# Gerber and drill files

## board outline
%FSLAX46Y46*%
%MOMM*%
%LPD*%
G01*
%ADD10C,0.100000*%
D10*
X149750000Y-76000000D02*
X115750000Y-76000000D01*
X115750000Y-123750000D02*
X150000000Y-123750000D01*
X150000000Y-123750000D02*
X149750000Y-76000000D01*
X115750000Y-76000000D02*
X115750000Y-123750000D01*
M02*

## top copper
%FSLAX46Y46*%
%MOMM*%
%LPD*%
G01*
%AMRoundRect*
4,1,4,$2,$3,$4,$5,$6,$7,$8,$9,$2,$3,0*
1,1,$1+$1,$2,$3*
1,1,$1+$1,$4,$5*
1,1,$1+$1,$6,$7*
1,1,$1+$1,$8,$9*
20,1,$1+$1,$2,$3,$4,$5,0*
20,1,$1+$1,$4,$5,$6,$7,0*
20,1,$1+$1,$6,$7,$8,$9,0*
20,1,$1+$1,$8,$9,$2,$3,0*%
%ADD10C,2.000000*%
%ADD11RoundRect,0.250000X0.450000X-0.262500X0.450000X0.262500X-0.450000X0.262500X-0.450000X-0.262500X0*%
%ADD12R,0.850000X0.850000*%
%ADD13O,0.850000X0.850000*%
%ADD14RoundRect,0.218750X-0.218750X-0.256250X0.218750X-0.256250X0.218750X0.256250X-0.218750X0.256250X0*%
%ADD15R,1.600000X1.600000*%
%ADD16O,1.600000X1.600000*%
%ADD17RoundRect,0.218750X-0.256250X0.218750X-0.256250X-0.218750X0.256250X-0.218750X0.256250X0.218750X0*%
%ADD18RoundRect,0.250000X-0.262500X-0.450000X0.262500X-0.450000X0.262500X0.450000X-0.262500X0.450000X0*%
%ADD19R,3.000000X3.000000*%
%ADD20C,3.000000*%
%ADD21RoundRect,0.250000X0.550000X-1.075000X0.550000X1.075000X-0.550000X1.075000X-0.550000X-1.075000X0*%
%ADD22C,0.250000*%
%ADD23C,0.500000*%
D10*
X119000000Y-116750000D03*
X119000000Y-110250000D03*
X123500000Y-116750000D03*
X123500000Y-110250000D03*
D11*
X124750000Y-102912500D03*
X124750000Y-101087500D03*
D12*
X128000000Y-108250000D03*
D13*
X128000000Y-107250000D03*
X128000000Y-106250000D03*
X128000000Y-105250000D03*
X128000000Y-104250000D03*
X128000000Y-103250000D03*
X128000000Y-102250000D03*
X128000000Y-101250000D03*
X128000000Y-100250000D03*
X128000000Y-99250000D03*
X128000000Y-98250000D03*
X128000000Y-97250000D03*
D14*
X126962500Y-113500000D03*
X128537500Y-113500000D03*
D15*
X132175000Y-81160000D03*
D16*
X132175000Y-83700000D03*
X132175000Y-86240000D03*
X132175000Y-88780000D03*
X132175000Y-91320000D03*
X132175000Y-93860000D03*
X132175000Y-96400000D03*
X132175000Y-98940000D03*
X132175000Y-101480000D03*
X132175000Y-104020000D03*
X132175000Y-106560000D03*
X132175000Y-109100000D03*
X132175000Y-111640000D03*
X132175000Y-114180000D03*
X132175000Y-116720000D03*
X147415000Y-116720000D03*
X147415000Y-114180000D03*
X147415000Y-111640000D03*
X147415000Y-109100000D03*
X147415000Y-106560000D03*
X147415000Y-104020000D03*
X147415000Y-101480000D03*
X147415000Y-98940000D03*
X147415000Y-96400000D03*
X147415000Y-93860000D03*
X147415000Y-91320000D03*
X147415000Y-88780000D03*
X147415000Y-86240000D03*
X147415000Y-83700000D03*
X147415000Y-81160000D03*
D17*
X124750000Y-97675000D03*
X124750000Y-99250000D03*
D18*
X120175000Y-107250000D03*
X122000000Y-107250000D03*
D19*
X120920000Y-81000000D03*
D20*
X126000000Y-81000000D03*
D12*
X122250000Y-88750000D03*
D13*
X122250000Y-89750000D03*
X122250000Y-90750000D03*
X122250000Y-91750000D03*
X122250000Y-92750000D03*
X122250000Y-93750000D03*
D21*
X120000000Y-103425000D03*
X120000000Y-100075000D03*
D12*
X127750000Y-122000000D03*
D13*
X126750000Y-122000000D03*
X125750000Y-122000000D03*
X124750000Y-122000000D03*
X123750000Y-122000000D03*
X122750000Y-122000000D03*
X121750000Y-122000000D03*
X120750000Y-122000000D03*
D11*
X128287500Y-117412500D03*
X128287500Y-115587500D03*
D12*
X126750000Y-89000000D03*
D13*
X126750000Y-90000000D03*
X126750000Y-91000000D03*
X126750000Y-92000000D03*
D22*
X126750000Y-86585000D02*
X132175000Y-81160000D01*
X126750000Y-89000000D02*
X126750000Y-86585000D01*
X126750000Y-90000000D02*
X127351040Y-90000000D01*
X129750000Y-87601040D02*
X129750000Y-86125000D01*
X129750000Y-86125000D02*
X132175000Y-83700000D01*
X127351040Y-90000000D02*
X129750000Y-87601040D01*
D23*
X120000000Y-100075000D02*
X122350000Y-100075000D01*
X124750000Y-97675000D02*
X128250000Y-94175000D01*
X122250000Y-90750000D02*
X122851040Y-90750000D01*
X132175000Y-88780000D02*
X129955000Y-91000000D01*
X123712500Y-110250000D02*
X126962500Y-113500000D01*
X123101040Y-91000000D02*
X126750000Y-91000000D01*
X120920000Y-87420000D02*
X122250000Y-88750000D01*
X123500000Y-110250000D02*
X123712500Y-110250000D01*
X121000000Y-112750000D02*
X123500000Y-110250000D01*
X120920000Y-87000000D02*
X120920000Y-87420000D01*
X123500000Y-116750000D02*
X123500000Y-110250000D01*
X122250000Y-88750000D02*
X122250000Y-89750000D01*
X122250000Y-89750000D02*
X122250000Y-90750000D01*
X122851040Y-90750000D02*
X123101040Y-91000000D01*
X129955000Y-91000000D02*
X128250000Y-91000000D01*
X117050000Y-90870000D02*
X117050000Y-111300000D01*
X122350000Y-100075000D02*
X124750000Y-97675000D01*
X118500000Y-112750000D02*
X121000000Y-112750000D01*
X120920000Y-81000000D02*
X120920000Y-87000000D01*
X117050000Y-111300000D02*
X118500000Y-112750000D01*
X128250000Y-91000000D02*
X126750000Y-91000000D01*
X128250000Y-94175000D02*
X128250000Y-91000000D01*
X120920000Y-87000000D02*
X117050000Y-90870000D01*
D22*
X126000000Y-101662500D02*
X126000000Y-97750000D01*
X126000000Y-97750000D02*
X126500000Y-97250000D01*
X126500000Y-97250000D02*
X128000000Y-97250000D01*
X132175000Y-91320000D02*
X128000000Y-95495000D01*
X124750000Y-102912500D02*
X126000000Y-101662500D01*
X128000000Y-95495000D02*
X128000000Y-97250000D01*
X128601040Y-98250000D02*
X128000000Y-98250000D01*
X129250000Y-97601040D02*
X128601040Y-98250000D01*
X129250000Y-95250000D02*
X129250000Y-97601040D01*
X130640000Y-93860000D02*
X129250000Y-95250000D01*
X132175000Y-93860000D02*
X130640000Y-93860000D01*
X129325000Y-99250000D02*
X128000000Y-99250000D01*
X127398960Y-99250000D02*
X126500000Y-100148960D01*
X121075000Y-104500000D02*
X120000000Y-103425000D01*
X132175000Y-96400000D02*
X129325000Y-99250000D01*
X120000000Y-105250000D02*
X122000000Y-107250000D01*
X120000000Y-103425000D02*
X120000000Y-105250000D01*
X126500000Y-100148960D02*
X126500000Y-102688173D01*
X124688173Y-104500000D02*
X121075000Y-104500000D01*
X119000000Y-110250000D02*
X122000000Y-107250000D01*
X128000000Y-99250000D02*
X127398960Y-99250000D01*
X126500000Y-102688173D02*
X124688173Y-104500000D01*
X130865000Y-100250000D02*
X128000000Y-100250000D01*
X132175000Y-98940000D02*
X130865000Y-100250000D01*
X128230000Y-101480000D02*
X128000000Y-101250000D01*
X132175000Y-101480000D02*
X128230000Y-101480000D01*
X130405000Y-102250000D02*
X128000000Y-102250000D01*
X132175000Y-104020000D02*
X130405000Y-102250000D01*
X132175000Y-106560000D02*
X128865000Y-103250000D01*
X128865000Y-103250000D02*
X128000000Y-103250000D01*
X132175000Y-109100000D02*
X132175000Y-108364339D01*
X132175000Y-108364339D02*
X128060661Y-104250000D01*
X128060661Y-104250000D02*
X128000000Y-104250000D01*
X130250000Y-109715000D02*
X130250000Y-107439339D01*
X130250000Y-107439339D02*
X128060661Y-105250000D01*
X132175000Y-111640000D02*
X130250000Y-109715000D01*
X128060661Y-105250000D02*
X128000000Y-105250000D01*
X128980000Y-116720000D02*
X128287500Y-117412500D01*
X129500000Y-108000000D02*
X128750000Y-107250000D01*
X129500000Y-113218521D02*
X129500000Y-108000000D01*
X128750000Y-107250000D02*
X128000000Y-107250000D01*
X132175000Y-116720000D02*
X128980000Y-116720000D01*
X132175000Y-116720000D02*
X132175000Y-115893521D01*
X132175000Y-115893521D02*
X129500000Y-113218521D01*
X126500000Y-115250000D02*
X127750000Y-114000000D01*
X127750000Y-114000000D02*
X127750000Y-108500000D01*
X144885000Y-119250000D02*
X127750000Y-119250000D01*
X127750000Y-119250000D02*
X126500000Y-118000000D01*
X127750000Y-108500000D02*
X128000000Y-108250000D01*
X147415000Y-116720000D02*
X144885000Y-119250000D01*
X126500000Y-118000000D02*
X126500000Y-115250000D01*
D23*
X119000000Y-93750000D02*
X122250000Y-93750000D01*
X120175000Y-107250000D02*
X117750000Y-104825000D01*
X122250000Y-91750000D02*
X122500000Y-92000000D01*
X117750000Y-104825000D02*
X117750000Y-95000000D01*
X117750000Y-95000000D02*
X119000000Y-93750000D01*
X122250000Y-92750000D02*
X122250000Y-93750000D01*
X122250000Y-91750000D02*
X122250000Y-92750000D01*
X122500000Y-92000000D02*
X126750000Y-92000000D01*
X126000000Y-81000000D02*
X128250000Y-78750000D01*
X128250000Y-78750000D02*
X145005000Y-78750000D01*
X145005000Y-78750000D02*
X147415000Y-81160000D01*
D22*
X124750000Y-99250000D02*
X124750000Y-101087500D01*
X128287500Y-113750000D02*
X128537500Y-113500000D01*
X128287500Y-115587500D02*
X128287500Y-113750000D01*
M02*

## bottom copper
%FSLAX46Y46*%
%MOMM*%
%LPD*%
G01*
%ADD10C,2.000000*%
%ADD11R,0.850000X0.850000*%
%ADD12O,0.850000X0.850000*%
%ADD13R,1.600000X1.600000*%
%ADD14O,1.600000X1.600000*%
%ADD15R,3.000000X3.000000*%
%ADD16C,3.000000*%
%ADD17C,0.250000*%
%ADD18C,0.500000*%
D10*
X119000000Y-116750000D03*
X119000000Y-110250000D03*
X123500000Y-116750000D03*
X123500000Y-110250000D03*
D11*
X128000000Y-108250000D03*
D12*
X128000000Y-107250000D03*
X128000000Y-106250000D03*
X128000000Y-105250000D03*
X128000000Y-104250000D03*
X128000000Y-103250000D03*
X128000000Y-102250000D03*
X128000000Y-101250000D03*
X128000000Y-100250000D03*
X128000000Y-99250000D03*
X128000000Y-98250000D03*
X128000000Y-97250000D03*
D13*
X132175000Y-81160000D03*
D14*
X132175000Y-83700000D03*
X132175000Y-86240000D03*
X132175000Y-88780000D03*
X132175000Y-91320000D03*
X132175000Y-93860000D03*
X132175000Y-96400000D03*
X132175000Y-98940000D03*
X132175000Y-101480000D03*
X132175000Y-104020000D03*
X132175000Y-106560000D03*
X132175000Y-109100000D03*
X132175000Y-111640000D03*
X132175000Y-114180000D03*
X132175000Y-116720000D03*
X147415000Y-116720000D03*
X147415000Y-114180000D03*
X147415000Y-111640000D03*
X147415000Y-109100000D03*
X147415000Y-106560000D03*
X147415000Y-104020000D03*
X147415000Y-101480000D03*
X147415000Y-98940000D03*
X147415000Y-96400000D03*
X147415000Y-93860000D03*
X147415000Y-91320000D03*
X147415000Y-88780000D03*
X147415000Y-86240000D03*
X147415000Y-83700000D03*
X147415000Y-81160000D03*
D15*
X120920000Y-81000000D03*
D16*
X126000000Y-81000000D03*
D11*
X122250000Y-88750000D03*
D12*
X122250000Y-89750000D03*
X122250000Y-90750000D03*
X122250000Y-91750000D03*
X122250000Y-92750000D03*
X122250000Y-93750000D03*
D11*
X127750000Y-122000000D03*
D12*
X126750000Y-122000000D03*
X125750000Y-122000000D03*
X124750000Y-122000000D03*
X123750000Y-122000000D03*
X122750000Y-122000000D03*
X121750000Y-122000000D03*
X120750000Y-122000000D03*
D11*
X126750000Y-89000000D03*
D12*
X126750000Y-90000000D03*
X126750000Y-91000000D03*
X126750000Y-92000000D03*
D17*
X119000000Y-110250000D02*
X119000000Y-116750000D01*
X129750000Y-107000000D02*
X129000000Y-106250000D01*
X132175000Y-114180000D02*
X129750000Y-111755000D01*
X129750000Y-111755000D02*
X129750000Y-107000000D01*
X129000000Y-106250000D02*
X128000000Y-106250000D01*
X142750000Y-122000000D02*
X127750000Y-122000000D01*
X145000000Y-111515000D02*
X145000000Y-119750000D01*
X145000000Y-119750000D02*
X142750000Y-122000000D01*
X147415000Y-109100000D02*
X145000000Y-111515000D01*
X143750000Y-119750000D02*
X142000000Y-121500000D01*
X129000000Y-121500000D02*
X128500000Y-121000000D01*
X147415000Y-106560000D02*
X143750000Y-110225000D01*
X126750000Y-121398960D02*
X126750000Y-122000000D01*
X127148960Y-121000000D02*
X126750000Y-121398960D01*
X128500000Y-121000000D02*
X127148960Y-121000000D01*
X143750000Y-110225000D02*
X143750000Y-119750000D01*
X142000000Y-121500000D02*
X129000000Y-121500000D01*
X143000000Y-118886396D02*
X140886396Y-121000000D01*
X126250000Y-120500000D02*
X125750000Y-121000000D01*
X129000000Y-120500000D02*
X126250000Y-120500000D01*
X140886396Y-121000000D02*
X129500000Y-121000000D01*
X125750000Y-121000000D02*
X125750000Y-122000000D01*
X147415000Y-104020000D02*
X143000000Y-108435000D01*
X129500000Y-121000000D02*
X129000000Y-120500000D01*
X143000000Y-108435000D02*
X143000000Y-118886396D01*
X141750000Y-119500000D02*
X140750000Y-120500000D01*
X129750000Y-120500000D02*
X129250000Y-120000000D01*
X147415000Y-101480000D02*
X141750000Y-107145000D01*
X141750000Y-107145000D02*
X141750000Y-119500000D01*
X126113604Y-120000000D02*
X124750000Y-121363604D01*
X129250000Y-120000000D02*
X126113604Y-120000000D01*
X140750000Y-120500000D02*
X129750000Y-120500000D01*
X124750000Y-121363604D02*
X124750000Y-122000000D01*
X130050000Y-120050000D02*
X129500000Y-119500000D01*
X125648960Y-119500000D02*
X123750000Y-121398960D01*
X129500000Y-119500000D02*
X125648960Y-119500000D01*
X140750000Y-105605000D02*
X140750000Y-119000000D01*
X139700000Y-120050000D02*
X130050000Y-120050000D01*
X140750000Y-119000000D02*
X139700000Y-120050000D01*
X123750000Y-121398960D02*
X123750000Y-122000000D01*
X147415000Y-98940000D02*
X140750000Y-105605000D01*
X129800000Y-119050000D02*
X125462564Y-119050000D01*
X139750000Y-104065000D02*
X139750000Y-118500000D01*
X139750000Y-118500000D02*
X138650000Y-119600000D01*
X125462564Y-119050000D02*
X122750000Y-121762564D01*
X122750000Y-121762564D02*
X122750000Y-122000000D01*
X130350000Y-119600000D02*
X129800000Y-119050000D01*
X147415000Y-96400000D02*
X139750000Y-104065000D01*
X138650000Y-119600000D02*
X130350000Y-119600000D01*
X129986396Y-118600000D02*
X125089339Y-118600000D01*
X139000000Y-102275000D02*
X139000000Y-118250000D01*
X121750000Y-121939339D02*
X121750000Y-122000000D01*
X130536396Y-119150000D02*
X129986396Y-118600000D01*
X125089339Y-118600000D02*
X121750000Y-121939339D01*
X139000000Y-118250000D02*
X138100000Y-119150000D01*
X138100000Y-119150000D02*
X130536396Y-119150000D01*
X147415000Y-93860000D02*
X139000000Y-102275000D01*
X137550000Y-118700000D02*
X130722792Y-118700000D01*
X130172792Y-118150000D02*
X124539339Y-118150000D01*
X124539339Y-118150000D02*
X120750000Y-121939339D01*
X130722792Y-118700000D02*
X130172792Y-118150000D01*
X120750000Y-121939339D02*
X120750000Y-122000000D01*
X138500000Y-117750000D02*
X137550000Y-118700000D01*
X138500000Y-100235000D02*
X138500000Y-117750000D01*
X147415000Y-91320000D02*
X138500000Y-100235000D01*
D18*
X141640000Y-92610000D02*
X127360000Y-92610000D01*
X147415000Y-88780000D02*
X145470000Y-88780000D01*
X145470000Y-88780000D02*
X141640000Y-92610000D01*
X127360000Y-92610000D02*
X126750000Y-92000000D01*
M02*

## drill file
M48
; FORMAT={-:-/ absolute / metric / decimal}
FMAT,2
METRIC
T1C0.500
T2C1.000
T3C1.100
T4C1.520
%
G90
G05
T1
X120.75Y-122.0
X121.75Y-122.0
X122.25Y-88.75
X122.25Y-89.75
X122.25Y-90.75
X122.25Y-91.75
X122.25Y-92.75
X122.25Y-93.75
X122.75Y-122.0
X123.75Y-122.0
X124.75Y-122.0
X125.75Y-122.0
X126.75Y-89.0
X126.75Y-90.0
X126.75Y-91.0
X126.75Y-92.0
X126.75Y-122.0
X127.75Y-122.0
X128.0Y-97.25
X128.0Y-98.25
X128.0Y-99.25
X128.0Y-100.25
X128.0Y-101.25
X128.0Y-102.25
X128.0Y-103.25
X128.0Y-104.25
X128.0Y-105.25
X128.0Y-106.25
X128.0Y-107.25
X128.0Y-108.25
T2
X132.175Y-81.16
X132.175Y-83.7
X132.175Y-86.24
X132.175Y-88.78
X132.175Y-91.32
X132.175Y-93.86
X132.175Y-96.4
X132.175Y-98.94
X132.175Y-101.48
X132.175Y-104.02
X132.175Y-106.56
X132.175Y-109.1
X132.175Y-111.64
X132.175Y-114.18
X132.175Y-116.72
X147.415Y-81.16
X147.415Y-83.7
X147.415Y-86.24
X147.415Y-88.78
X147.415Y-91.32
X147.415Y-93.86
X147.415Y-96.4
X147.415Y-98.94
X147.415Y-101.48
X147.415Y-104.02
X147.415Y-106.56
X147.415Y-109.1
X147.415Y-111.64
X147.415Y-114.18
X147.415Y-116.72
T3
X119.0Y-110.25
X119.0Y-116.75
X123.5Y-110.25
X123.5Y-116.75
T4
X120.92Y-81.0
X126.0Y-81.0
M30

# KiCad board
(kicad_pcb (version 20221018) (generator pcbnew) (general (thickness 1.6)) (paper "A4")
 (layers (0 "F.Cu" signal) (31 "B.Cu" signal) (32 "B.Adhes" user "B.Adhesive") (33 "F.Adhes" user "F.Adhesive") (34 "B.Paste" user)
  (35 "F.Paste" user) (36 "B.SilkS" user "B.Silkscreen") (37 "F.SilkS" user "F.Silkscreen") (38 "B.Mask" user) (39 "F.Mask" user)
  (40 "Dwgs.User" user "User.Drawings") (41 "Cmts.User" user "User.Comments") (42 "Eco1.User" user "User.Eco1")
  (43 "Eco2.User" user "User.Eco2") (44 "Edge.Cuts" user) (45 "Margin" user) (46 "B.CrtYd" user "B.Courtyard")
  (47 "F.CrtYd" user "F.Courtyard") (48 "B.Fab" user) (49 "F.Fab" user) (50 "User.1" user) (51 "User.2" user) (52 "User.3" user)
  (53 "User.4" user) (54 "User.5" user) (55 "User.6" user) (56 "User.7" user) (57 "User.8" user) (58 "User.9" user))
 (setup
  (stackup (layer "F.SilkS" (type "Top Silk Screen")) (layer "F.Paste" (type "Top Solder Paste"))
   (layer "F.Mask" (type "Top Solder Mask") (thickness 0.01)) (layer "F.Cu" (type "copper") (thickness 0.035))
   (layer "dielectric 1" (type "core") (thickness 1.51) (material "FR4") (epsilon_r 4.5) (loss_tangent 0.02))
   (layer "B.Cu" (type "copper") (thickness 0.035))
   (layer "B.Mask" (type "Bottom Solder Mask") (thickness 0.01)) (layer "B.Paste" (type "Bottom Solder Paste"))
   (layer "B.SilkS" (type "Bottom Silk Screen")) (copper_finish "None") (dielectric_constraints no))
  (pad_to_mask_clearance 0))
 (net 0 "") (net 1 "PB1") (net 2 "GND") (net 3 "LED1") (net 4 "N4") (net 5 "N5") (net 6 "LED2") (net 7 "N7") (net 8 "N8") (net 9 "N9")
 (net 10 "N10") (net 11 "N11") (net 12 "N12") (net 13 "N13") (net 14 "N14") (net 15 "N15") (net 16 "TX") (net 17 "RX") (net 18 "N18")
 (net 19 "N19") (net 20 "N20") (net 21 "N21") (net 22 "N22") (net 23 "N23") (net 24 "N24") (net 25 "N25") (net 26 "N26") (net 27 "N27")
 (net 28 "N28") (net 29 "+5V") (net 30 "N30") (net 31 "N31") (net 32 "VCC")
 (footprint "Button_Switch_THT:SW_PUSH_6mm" (layer "F.Cu") (at 119 116.75 90)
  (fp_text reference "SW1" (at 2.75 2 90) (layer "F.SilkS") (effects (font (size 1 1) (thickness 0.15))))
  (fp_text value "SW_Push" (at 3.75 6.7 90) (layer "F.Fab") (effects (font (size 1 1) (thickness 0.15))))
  (pad "1" thru_hole circle (at 0 0 180) (size 2 2) (drill 1.1) (layers "*.Cu" "*.Mask") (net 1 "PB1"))
  (pad "1" thru_hole circle (at 6.5 0 180) (size 2 2) (drill 1.1) (layers "*.Cu" "*.Mask") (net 1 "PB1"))
  (pad "2" thru_hole circle (at 0 4.5 180) (size 2 2) (drill 1.1) (layers "*.Cu" "*.Mask") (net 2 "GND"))
  (pad "2" thru_hole circle (at 6.5 4.5 180) (size 2 2) (drill 1.1) (layers "*.Cu" "*.Mask") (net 2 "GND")))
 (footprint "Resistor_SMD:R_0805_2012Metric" (layer "F.Cu") (at 124.75 102 90)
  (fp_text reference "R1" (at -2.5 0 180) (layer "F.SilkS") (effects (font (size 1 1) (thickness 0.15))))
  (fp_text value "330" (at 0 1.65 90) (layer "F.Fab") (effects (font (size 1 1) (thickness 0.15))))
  (pad "1" smd roundrect (at -0.9125 0 90) (size 1.025 1.4) (layers "F.Cu" "F.Paste" "F.Mask") (roundrect_rratio 0.243902) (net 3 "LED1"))
  (pad "2" smd roundrect (at 0.9125 0 90) (size 1.025 1.4) (layers "F.Cu" "F.Paste" "F.Mask") (roundrect_rratio 0.243902) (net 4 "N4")))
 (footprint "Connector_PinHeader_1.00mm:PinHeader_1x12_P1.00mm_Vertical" (layer "F.Cu") (at 128 108.25 180)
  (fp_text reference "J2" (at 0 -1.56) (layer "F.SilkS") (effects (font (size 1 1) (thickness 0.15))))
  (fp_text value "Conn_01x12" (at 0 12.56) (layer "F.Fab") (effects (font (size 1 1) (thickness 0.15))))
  (pad "1" thru_hole rect (at 0 0 180) (size 0.85 0.85) (drill 0.5) (layers "*.Cu" "*.Mask") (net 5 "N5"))
  (pad "2" thru_hole oval (at 0 1 180) (size 0.85 0.85) (drill 0.5) (layers "*.Cu" "*.Mask") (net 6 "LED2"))
  (pad "3" thru_hole oval (at 0 2 180) (size 0.85 0.85) (drill 0.5) (layers "*.Cu" "*.Mask") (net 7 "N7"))
  (pad "4" thru_hole oval (at 0 3 180) (size 0.85 0.85) (drill 0.5) (layers "*.Cu" "*.Mask") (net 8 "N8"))
  (pad "5" thru_hole oval (at 0 4 180) (size 0.85 0.85) (drill 0.5) (layers "*.Cu" "*.Mask") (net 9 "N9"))
  (pad "6" thru_hole oval (at 0 5 180) (size 0.85 0.85) (drill 0.5) (layers "*.Cu" "*.Mask") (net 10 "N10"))
  (pad "7" thru_hole oval (at 0 6 180) (size 0.85 0.85) (drill 0.5) (layers "*.Cu" "*.Mask") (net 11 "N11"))
  (pad "8" thru_hole oval (at 0 7 180) (size 0.85 0.85) (drill 0.5) (layers "*.Cu" "*.Mask") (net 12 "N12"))
  (pad "9" thru_hole oval (at 0 8 180) (size 0.85 0.85) (drill 0.5) (layers "*.Cu" "*.Mask") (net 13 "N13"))
  (pad "10" thru_hole oval (at 0 9 180) (size 0.85 0.85) (drill 0.5) (layers "*.Cu" "*.Mask") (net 1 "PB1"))
  (pad "11" thru_hole oval (at 0 10 180) (size 0.85 0.85) (drill 0.5) (layers "*.Cu" "*.Mask") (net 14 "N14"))
  (pad "12" thru_hole oval (at 0 11 180) (size 0.85 0.85) (drill 0.5) (layers "*.Cu" "*.Mask") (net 3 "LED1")))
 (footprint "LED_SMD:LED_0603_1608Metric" (layer "F.Cu") (at 127.75 113.5)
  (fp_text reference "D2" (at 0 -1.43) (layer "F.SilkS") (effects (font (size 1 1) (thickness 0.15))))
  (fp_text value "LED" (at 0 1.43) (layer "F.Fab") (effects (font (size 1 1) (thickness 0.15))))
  (pad "1" smd roundrect (at -0.7875 0) (size 0.875 0.95) (layers "F.Cu" "F.Paste" "F.Mask") (roundrect_rratio 0.25) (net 2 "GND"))
  (pad "2" smd roundrect (at 0.7875 0) (size 0.875 0.95) (layers "F.Cu" "F.Paste" "F.Mask") (roundrect_rratio 0.25) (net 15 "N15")))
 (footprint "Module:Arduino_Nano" (layer "F.Cu") (at 132.175 81.16)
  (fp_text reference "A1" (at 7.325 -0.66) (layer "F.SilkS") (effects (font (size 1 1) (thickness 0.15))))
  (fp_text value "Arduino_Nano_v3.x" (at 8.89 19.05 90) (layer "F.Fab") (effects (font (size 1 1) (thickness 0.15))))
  (pad "1" thru_hole rect (at 0 0) (size 1.6 1.6) (drill 1) (layers "*.Cu" "*.Mask") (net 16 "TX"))
  (pad "2" thru_hole oval (at 0 2.54) (size 1.6 1.6) (drill 1) (layers "*.Cu" "*.Mask") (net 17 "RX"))
  (pad "3" thru_hole oval (at 0 5.08) (size 1.6 1.6) (drill 1) (layers "*.Cu" "*.Mask") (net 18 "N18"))
  (pad "4" thru_hole oval (at 0 7.62) (size 1.6 1.6) (drill 1) (layers "*.Cu" "*.Mask") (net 2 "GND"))
  (pad "5" thru_hole oval (at 0 10.16) (size 1.6 1.6) (drill 1) (layers "*.Cu" "*.Mask") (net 3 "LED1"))
  (pad "6" thru_hole oval (at 0 12.7) (size 1.6 1.6) (drill 1) (layers "*.Cu" "*.Mask") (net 14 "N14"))
  (pad "7" thru_hole oval (at 0 15.24) (size 1.6 1.6) (drill 1) (layers "*.Cu" "*.Mask") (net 1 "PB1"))
  (pad "8" thru_hole oval (at 0 17.78) (size 1.6 1.6) (drill 1) (layers "*.Cu" "*.Mask") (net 13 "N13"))
  (pad "9" thru_hole oval (at 0 20.32) (size 1.6 1.6) (drill 1) (layers "*.Cu" "*.Mask") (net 12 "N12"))
  (pad "10" thru_hole oval (at 0 22.86) (size 1.6 1.6) (drill 1) (layers "*.Cu" "*.Mask") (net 11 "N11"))
  (pad "11" thru_hole oval (at 0 25.4) (size 1.6 1.6) (drill 1) (layers "*.Cu" "*.Mask") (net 10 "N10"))
  (pad "12" thru_hole oval (at 0 27.94) (size 1.6 1.6) (drill 1) (layers "*.Cu" "*.Mask") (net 9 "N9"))
  (pad "13" thru_hole oval (at 0 30.48) (size 1.6 1.6) (drill 1) (layers "*.Cu" "*.Mask") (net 8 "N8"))
  (pad "14" thru_hole oval (at 0 33.02) (size 1.6 1.6) (drill 1) (layers "*.Cu" "*.Mask") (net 7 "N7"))
  (pad "15" thru_hole oval (at 0 35.56) (size 1.6 1.6) (drill 1) (layers "*.Cu" "*.Mask") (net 6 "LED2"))
  (pad "16" thru_hole oval (at 15.24 35.56) (size 1.6 1.6) (drill 1) (layers "*.Cu" "*.Mask") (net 5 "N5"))
  (pad "17" thru_hole oval (at 15.24 33.02) (size 1.6 1.6) (drill 1) (layers "*.Cu" "*.Mask") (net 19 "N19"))
  (pad "18" thru_hole oval (at 15.24 30.48) (size 1.6 1.6) (drill 1) (layers "*.Cu" "*.Mask") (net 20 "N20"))
  (pad "19" thru_hole oval (at 15.24 27.94) (size 1.6 1.6) (drill 1) (layers "*.Cu" "*.Mask") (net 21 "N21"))
  (pad "20" thru_hole oval (at 15.24 25.4) (size 1.6 1.6) (drill 1) (layers "*.Cu" "*.Mask") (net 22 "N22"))
  (pad "21" thru_hole oval (at 15.24 22.86) (size 1.6 1.6) (drill 1) (layers "*.Cu" "*.Mask") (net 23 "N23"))
  (pad "22" thru_hole oval (at 15.24 20.32) (size 1.6 1.6) (drill 1) (layers "*.Cu" "*.Mask") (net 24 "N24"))
  (pad "23" thru_hole oval (at 15.24 17.78) (size 1.6 1.6) (drill 1) (layers "*.Cu" "*.Mask") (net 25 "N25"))
  (pad "24" thru_hole oval (at 15.24 15.24) (size 1.6 1.6) (drill 1) (layers "*.Cu" "*.Mask") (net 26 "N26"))
  (pad "25" thru_hole oval (at 15.24 12.7) (size 1.6 1.6) (drill 1) (layers "*.Cu" "*.Mask") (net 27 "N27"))
  (pad "26" thru_hole oval (at 15.24 10.16) (size 1.6 1.6) (drill 1) (layers "*.Cu" "*.Mask") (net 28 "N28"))
  (pad "27" thru_hole oval (at 15.24 7.62) (size 1.6 1.6) (drill 1) (layers "*.Cu" "*.Mask") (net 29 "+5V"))
  (pad "28" thru_hole oval (at 15.24 5.08) (size 1.6 1.6) (drill 1) (layers "*.Cu" "*.Mask") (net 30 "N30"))
  (pad "29" thru_hole oval (at 15.24 2.54) (size 1.6 1.6) (drill 1) (layers "*.Cu" "*.Mask") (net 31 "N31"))
  (pad "30" thru_hole oval (at 15.24 0) (size 1.6 1.6) (drill 1) (layers "*.Cu" "*.Mask") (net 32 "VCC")))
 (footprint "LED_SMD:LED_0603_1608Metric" (layer "F.Cu") (at 124.75 98.4625 -90)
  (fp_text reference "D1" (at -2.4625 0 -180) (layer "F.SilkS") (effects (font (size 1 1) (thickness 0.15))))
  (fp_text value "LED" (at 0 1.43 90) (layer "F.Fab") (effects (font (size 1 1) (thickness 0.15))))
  (pad "1" smd roundrect (at -0.7875 0 270) (size 0.875 0.95) (layers "F.Cu" "F.Paste" "F.Mask") (roundrect_rratio 0.25) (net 2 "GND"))
  (pad "2" smd roundrect (at 0.7875 0 270) (size 0.875 0.95) (layers "F.Cu" "F.Paste" "F.Mask") (roundrect_rratio 0.25) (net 4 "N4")))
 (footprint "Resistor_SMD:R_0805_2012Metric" (layer "F.Cu") (at 121.0875 107.25)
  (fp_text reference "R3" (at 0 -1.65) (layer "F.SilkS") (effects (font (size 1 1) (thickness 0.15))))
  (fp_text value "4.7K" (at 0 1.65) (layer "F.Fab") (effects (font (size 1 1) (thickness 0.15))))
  (pad "1" smd roundrect (at -0.9125 0) (size 1.025 1.4) (layers "F.Cu" "F.Paste" "F.Mask") (roundrect_rratio 0.243902) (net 29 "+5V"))
  (pad "2" smd roundrect (at 0.9125 0) (size 1.025 1.4) (layers "F.Cu" "F.Paste" "F.Mask") (roundrect_rratio 0.243902) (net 1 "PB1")))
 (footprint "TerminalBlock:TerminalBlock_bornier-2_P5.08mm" (layer "F.Cu") (at 120.92 81)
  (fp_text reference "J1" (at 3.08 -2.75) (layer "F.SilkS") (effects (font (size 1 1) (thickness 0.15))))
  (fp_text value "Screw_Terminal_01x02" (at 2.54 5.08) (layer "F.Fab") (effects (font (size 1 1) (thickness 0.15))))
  (pad "1" thru_hole rect (at 0 0) (size 3 3) (drill 1.52) (layers "*.Cu" "*.Mask") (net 2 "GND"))
  (pad "2" thru_hole circle (at 5.08 0) (size 3 3) (drill 1.52) (layers "*.Cu" "*.Mask") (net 32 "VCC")))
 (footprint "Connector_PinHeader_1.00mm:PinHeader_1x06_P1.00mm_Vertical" (layer "F.Cu") (at 122.25 88.75)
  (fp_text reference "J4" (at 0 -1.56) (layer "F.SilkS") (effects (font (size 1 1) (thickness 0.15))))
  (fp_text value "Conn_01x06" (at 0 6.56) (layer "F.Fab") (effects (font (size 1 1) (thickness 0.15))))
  (pad "1" thru_hole rect (at 0 0) (size 0.85 0.85) (drill 0.5) (layers "*.Cu" "*.Mask") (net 2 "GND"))
  (pad "2" thru_hole oval (at 0 1) (size 0.85 0.85) (drill 0.5) (layers "*.Cu" "*.Mask") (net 2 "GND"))
  (pad "3" thru_hole oval (at 0 2) (size 0.85 0.85) (drill 0.5) (layers "*.Cu" "*.Mask") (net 2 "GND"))
  (pad "4" thru_hole oval (at 0 3) (size 0.85 0.85) (drill 0.5) (layers "*.Cu" "*.Mask") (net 29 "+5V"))
  (pad "5" thru_hole oval (at 0 4) (size 0.85 0.85) (drill 0.5) (layers "*.Cu" "*.Mask") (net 29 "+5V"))
  (pad "6" thru_hole oval (at 0 5) (size 0.85 0.85) (drill 0.5) (layers "*.Cu" "*.Mask") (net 29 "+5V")))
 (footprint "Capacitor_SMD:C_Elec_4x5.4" (layer "F.Cu") (at 120 101.75 90)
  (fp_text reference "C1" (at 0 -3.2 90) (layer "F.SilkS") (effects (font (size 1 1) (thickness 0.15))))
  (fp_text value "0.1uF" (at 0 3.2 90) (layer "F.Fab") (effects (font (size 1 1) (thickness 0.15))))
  (pad "1" smd roundrect (at -1.675 0 90) (size 2.65 1.6) (layers "F.Cu" "F.Paste" "F.Mask") (roundrect_rratio 0.15625) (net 1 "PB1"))
  (pad "2" smd roundrect (at 1.675 0 90) (size 2.65 1.6) (layers "F.Cu" "F.Paste" "F.Mask") (roundrect_rratio 0.15625) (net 2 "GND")))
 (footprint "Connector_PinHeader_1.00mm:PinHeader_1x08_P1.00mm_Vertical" (layer "F.Cu") (at 127.75 122 -90)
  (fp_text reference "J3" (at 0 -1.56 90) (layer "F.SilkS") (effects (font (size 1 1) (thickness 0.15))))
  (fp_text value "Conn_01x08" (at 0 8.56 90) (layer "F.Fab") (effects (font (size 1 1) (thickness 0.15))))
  (pad "1" thru_hole rect (at 0 0 270) (size 0.85 0.85) (drill 0.5) (layers "*.Cu" "*.Mask") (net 21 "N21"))
  (pad "2" thru_hole oval (at 0 1 270) (size 0.85 0.85) (drill 0.5) (layers "*.Cu" "*.Mask") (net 22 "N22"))
  (pad "3" thru_hole oval (at 0 2 270) (size 0.85 0.85) (drill 0.5) (layers "*.Cu" "*.Mask") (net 23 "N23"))
  (pad "4" thru_hole oval (at 0 3 270) (size 0.85 0.85) (drill 0.5) (layers "*.Cu" "*.Mask") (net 24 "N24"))
  (pad "5" thru_hole oval (at 0 4 270) (size 0.85 0.85) (drill 0.5) (layers "*.Cu" "*.Mask") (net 25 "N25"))
  (pad "6" thru_hole oval (at 0 5 270) (size 0.85 0.85) (drill 0.5) (layers "*.Cu" "*.Mask") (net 26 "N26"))
  (pad "7" thru_hole oval (at 0 6 270) (size 0.85 0.85) (drill 0.5) (layers "*.Cu" "*.Mask") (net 27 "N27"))
  (pad "8" thru_hole oval (at 0 7 270) (size 0.85 0.85) (drill 0.5) (layers "*.Cu" "*.Mask") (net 28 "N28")))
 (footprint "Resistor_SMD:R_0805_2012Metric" (layer "F.Cu") (at 128.2875 116.5 90)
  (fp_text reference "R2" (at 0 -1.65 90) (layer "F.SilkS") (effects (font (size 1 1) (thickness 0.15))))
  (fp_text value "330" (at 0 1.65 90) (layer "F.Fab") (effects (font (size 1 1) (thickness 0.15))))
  (pad "1" smd roundrect (at -0.9125 0 90) (size 1.025 1.4) (layers "F.Cu" "F.Paste" "F.Mask") (roundrect_rratio 0.243902) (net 6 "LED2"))
  (pad "2" smd roundrect (at 0.9125 0 90) (size 1.025 1.4) (layers "F.Cu" "F.Paste" "F.Mask") (roundrect_rratio 0.243902) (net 15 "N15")))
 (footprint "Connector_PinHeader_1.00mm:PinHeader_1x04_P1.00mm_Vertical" (layer "F.Cu") (at 126.75 89)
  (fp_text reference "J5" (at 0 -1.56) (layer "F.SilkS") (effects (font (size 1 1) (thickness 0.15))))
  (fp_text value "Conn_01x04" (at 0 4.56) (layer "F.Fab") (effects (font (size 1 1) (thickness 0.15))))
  (pad "1" thru_hole rect (at 0 0) (size 0.85 0.85) (drill 0.5) (layers "*.Cu" "*.Mask") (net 16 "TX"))
  (pad "2" thru_hole oval (at 0 1) (size 0.85 0.85) (drill 0.5) (layers "*.Cu" "*.Mask") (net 17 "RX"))
  (pad "3" thru_hole oval (at 0 2) (size 0.85 0.85) (drill 0.5) (layers "*.Cu" "*.Mask") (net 2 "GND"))
  (pad "4" thru_hole oval (at 0 3) (size 0.85 0.85) (drill 0.5) (layers "*.Cu" "*.Mask") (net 29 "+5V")))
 (gr_line (start 149.75 76) (end 115.75 76) (stroke (width 0.1) (type default)) (layer "Edge.Cuts"))
 (gr_line (start 115.75 123.75) (end 150 123.75) (stroke (width 0.1) (type default)) (layer "Edge.Cuts"))
 (gr_line (start 150 123.75) (end 149.75 76) (stroke (width 0.1) (type default)) (layer "Edge.Cuts"))
 (gr_line (start 115.75 76) (end 115.75 123.75) (stroke (width 0.1) (type default)) (layer "Edge.Cuts"))
 (segment (start 126.75 86.585) (end 132.175 81.16) (width 0.25) (layer "F.Cu") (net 16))
 (segment (start 126.75 89) (end 126.75 86.585) (width 0.25) (layer "F.Cu") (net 16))
 (segment (start 126.75 90) (end 127.35104 90) (width 0.25) (layer "F.Cu") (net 17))
 (segment (start 129.75 87.60104) (end 129.75 86.125) (width 0.25) (layer "F.Cu") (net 17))
 (segment (start 129.75 86.125) (end 132.175 83.7) (width 0.25) (layer "F.Cu") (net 17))
 (segment (start 127.35104 90) (end 129.75 87.60104) (width 0.25) (layer "F.Cu") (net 17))
 (segment (start 120 100.075) (end 122.35 100.075) (width 0.5) (layer "F.Cu") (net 2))
 (segment (start 124.75 97.675) (end 128.25 94.175) (width 0.5) (layer "F.Cu") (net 2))
 (segment (start 122.25 90.75) (end 122.85104 90.75) (width 0.5) (layer "F.Cu") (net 2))
 (segment (start 132.175 88.78) (end 129.955 91) (width 0.5) (layer "F.Cu") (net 2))
 (segment (start 123.7125 110.25) (end 126.9625 113.5) (width 0.5) (layer "F.Cu") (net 2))
 (segment (start 123.10104 91) (end 126.75 91) (width 0.5) (layer "F.Cu") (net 2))
 (segment (start 120.92 87.42) (end 122.25 88.75) (width 0.5) (layer "F.Cu") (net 2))
 (segment (start 123.5 110.25) (end 123.7125 110.25) (width 0.5) (layer "F.Cu") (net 2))
 (segment (start 121 112.75) (end 123.5 110.25) (width 0.5) (layer "F.Cu") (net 2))
 (segment (start 120.92 87) (end 120.92 87.42) (width 0.5) (layer "F.Cu") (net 2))
 (segment (start 123.5 116.75) (end 123.5 110.25) (width 0.5) (layer "F.Cu") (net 2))
 (segment (start 122.25 88.75) (end 122.25 89.75) (width 0.5) (layer "F.Cu") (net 2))
 (segment (start 122.25 89.75) (end 122.25 90.75) (width 0.5) (layer "F.Cu") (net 2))
 (segment (start 122.85104 90.75) (end 123.10104 91) (width 0.5) (layer "F.Cu") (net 2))
 (segment (start 129.955 91) (end 128.25 91) (width 0.5) (layer "F.Cu") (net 2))
 (segment (start 117.05 90.87) (end 117.05 111.3) (width 0.5) (layer "F.Cu") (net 2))
 (segment (start 122.35 100.075) (end 124.75 97.675) (width 0.5) (layer "F.Cu") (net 2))
 (segment (start 118.5 112.75) (end 121 112.75) (width 0.5) (layer "F.Cu") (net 2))
 (segment (start 120.92 81) (end 120.92 87) (width 0.5) (layer "F.Cu") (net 2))
 (segment (start 117.05 111.3) (end 118.5 112.75) (width 0.5) (layer "F.Cu") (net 2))
 (segment (start 128.25 91) (end 126.75 91) (width 0.5) (layer "F.Cu") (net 2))
 (segment (start 128.25 94.175) (end 128.25 91) (width 0.5) (layer "F.Cu") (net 2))
 (segment (start 120.92 87) (end 117.05 90.87) (width 0.5) (layer "F.Cu") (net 2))
 (segment (start 126 101.6625) (end 126 97.75) (width 0.25) (layer "F.Cu") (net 3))
 (segment (start 126 97.75) (end 126.5 97.25) (width 0.25) (layer "F.Cu") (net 3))
 (segment (start 126.5 97.25) (end 128 97.25) (width 0.25) (layer "F.Cu") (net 3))
 (segment (start 132.175 91.32) (end 128 95.495) (width 0.25) (layer "F.Cu") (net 3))
 (segment (start 124.75 102.9125) (end 126 101.6625) (width 0.25) (layer "F.Cu") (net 3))
 (segment (start 128 95.495) (end 128 97.25) (width 0.25) (layer "F.Cu") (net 3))
 (segment (start 128.60104 98.25) (end 128 98.25) (width 0.25) (layer "F.Cu") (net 14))
 (segment (start 129.25 97.60104) (end 128.60104 98.25) (width 0.25) (layer "F.Cu") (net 14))
 (segment (start 129.25 95.25) (end 129.25 97.60104) (width 0.25) (layer "F.Cu") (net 14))
 (segment (start 130.64 93.86) (end 129.25 95.25) (width 0.25) (layer "F.Cu") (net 14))
 (segment (start 132.175 93.86) (end 130.64 93.86) (width 0.25) (layer "F.Cu") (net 14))
 (segment (start 129.325 99.25) (end 128 99.25) (width 0.25) (layer "F.Cu") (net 1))
 (segment (start 127.39896 99.25) (end 126.5 100.14896) (width 0.25) (layer "F.Cu") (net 1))
 (segment (start 121.075 104.5) (end 120 103.425) (width 0.25) (layer "F.Cu") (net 1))
 (segment (start 132.175 96.4) (end 129.325 99.25) (width 0.25) (layer "F.Cu") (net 1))
 (segment (start 120 105.25) (end 122 107.25) (width 0.25) (layer "F.Cu") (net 1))
 (segment (start 120 103.425) (end 120 105.25) (width 0.25) (layer "F.Cu") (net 1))
 (segment (start 126.5 100.14896) (end 126.5 102.688173) (width 0.25) (layer "F.Cu") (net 1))
 (segment (start 124.688173 104.5) (end 121.075 104.5) (width 0.25) (layer "F.Cu") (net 1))
 (segment (start 119 110.25) (end 122 107.25) (width 0.25) (layer "F.Cu") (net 1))
 (segment (start 128 99.25) (end 127.39896 99.25) (width 0.25) (layer "F.Cu") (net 1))
 (segment (start 126.5 102.688173) (end 124.688173 104.5) (width 0.25) (layer "F.Cu") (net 1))
 (segment (start 119 110.25) (end 119 116.75) (width 0.25) (layer "B.Cu") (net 1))
 (segment (start 130.865 100.25) (end 128 100.25) (width 0.25) (layer "F.Cu") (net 13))
 (segment (start 132.175 98.94) (end 130.865 100.25) (width 0.25) (layer "F.Cu") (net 13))
 (segment (start 128.23 101.48) (end 128 101.25) (width 0.25) (layer "F.Cu") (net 12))
 (segment (start 132.175 101.48) (end 128.23 101.48) (width 0.25) (layer "F.Cu") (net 12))
 (segment (start 130.405 102.25) (end 128 102.25) (width 0.25) (layer "F.Cu") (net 11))
 (segment (start 132.175 104.02) (end 130.405 102.25) (width 0.25) (layer "F.Cu") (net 11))
 (segment (start 132.175 106.56) (end 128.865 103.25) (width 0.25) (layer "F.Cu") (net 10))
 (segment (start 128.865 103.25) (end 128 103.25) (width 0.25) (layer "F.Cu") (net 10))
 (segment (start 132.175 109.1) (end 132.175 108.364339) (width 0.25) (layer "F.Cu") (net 9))
 (segment (start 132.175 108.364339) (end 128.060661 104.25) (width 0.25) (layer "F.Cu") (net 9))
 (segment (start 128.060661 104.25) (end 128 104.25) (width 0.25) (layer "F.Cu") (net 9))
 (segment (start 130.25 109.715) (end 130.25 107.439339) (width 0.25) (layer "F.Cu") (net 8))
 (segment (start 130.25 107.439339) (end 128.060661 105.25) (width 0.25) (layer "F.Cu") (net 8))
 (segment (start 132.175 111.64) (end 130.25 109.715) (width 0.25) (layer "F.Cu") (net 8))
 (segment (start 128.060661 105.25) (end 128 105.25) (width 0.25) (layer "F.Cu") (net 8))
 (segment (start 129.75 107) (end 129 106.25) (width 0.25) (layer "B.Cu") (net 7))
 (segment (start 132.175 114.18) (end 129.75 111.755) (width 0.25) (layer "B.Cu") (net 7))
 (segment (start 129.75 111.755) (end 129.75 107) (width 0.25) (layer "B.Cu") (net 7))
 (segment (start 129 106.25) (end 128 106.25) (width 0.25) (layer "B.Cu") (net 7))
 (segment (start 128.98 116.72) (end 128.2875 117.4125) (width 0.25) (layer "F.Cu") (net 6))
 (segment (start 129.5 108) (end 128.75 107.25) (width 0.25) (layer "F.Cu") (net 6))
 (segment (start 129.5 113.218521) (end 129.5 108) (width 0.25) (layer "F.Cu") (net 6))
 (segment (start 128.75 107.25) (end 128 107.25) (width 0.25) (layer "F.Cu") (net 6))
 (segment (start 132.175 116.72) (end 128.98 116.72) (width 0.25) (layer "F.Cu") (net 6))
 (segment (start 132.175 116.72) (end 132.175 115.893521) (width 0.25) (layer "F.Cu") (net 6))
 (segment (start 132.175 115.893521) (end 129.5 113.218521) (width 0.25) (layer "F.Cu") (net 6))
 (segment (start 126.5 115.25) (end 127.75 114) (width 0.25) (layer "F.Cu") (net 5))
 (segment (start 127.75 114) (end 127.75 108.5) (width 0.25) (layer "F.Cu") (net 5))
 (segment (start 144.885 119.25) (end 127.75 119.25) (width 0.25) (layer "F.Cu") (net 5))
 (segment (start 127.75 119.25) (end 126.5 118) (width 0.25) (layer "F.Cu") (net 5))
 (segment (start 127.75 108.5) (end 128 108.25) (width 0.25) (layer "F.Cu") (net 5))
 (segment (start 147.415 116.72) (end 144.885 119.25) (width 0.25) (layer "F.Cu") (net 5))
 (segment (start 126.5 118) (end 126.5 115.25) (width 0.25) (layer "F.Cu") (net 5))
 (segment (start 142.75 122) (end 127.75 122) (width 0.25) (layer "B.Cu") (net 21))
 (segment (start 145 111.515) (end 145 119.75) (width 0.25) (layer "B.Cu") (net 21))
 (segment (start 145 119.75) (end 142.75 122) (width 0.25) (layer "B.Cu") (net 21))
 (segment (start 147.415 109.1) (end 145 111.515) (width 0.25) (layer "B.Cu") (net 21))
 (segment (start 143.75 119.75) (end 142 121.5) (width 0.25) (layer "B.Cu") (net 22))
 (segment (start 129 121.5) (end 128.5 121) (width 0.25) (layer "B.Cu") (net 22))
 (segment (start 147.415 106.56) (end 143.75 110.225) (width 0.25) (layer "B.Cu") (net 22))
 (segment (start 126.75 121.39896) (end 126.75 122) (width 0.25) (layer "B.Cu") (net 22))
 (segment (start 127.14896 121) (end 126.75 121.39896) (width 0.25) (layer "B.Cu") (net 22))
 (segment (start 128.5 121) (end 127.14896 121) (width 0.25) (layer "B.Cu") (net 22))
 (segment (start 143.75 110.225) (end 143.75 119.75) (width 0.25) (layer "B.Cu") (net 22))
 (segment (start 142 121.5) (end 129 121.5) (width 0.25) (layer "B.Cu") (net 22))
 (segment (start 143 118.886396) (end 140.886396 121) (width 0.25) (layer "B.Cu") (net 23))
 (segment (start 126.25 120.5) (end 125.75 121) (width 0.25) (layer "B.Cu") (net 23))
 (segment (start 129 120.5) (end 126.25 120.5) (width 0.25) (layer "B.Cu") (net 23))
 (segment (start 140.886396 121) (end 129.5 121) (width 0.25) (layer "B.Cu") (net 23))
 (segment (start 125.75 121) (end 125.75 122) (width 0.25) (layer "B.Cu") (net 23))
 (segment (start 147.415 104.02) (end 143 108.435) (width 0.25) (layer "B.Cu") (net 23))
 (segment (start 129.5 121) (end 129 120.5) (width 0.25) (layer "B.Cu") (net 23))
 (segment (start 143 108.435) (end 143 118.886396) (width 0.25) (layer "B.Cu") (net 23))
 (segment (start 141.75 119.5) (end 140.75 120.5) (width 0.25) (layer "B.Cu") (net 24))
 (segment (start 129.75 120.5) (end 129.25 120) (width 0.25) (layer "B.Cu") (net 24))
 (segment (start 147.415 101.48) (end 141.75 107.145) (width 0.25) (layer "B.Cu") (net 24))
 (segment (start 141.75 107.145) (end 141.75 119.5) (width 0.25) (layer "B.Cu") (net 24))
 (segment (start 126.113604 120) (end 124.75 121.363604) (width 0.25) (layer "B.Cu") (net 24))
 (segment (start 129.25 120) (end 126.113604 120) (width 0.25) (layer "B.Cu") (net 24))
 (segment (start 140.75 120.5) (end 129.75 120.5) (width 0.25) (layer "B.Cu") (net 24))
 (segment (start 124.75 121.363604) (end 124.75 122) (width 0.25) (layer "B.Cu") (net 24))
 (segment (start 130.05 120.05) (end 129.5 119.5) (width 0.25) (layer "B.Cu") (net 25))
 (segment (start 125.64896 119.5) (end 123.75 121.39896) (width 0.25) (layer "B.Cu") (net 25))
 (segment (start 129.5 119.5) (end 125.64896 119.5) (width 0.25) (layer "B.Cu") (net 25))
 (segment (start 140.75 105.605) (end 140.75 119) (width 0.25) (layer "B.Cu") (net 25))
 (segment (start 139.7 120.05) (end 130.05 120.05) (width 0.25) (layer "B.Cu") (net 25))
 (segment (start 140.75 119) (end 139.7 120.05) (width 0.25) (layer "B.Cu") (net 25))
 (segment (start 123.75 121.39896) (end 123.75 122) (width 0.25) (layer "B.Cu") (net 25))
 (segment (start 147.415 98.94) (end 140.75 105.605) (width 0.25) (layer "B.Cu") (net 25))
 (segment (start 129.8 119.05) (end 125.462564 119.05) (width 0.25) (layer "B.Cu") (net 26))
 (segment (start 139.75 104.065) (end 139.75 118.5) (width 0.25) (layer "B.Cu") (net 26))
 (segment (start 139.75 118.5) (end 138.65 119.6) (width 0.25) (layer "B.Cu") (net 26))
 (segment (start 125.462564 119.05) (end 122.75 121.762564) (width 0.25) (layer "B.Cu") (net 26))
 (segment (start 122.75 121.762564) (end 122.75 122) (width 0.25) (layer "B.Cu") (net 26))
 (segment (start 130.35 119.6) (end 129.8 119.05) (width 0.25) (layer "B.Cu") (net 26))
 (segment (start 147.415 96.4) (end 139.75 104.065) (width 0.25) (layer "B.Cu") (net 26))
 (segment (start 138.65 119.6) (end 130.35 119.6) (width 0.25) (layer "B.Cu") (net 26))
 (segment (start 129.986396 118.6) (end 125.089339 118.6) (width 0.25) (layer "B.Cu") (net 27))
 (segment (start 139 102.275) (end 139 118.25) (width 0.25) (layer "B.Cu") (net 27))
 (segment (start 121.75 121.939339) (end 121.75 122) (width 0.25) (layer "B.Cu") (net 27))
 (segment (start 130.536396 119.15) (end 129.986396 118.6) (width 0.25) (layer "B.Cu") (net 27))
 (segment (start 125.089339 118.6) (end 121.75 121.939339) (width 0.25) (layer "B.Cu") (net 27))
 (segment (start 139 118.25) (end 138.1 119.15) (width 0.25) (layer "B.Cu") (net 27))
 (segment (start 138.1 119.15) (end 130.536396 119.15) (width 0.25) (layer "B.Cu") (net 27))
 (segment (start 147.415 93.86) (end 139 102.275) (width 0.25) (layer "B.Cu") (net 27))
 (segment (start 137.55 118.7) (end 130.722792 118.7) (width 0.25) (layer "B.Cu") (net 28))
 (segment (start 130.172792 118.15) (end 124.539339 118.15) (width 0.25) (layer "B.Cu") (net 28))
 (segment (start 124.539339 118.15) (end 120.75 121.939339) (width 0.25) (layer "B.Cu") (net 28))
 (segment (start 130.722792 118.7) (end 130.172792 118.15) (width 0.25) (layer "B.Cu") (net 28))
 (segment (start 120.75 121.939339) (end 120.75 122) (width 0.25) (layer "B.Cu") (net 28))
 (segment (start 138.5 117.75) (end 137.55 118.7) (width 0.25) (layer "B.Cu") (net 28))
 (segment (start 138.5 100.235) (end 138.5 117.75) (width 0.25) (layer "B.Cu") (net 28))
 (segment (start 147.415 91.32) (end 138.5 100.235) (width 0.25) (layer "B.Cu") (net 28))
 (segment (start 119 93.75) (end 122.25 93.75) (width 0.5) (layer "F.Cu") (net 29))
 (segment (start 120.175 107.25) (end 117.75 104.825) (width 0.5) (layer "F.Cu") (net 29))
 (segment (start 122.25 91.75) (end 122.5 92) (width 0.5) (layer "F.Cu") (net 29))
 (segment (start 117.75 104.825) (end 117.75 95) (width 0.5) (layer "F.Cu") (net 29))
 (segment (start 117.75 95) (end 119 93.75) (width 0.5) (layer "F.Cu") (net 29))
 (segment (start 122.25 92.75) (end 122.25 93.75) (width 0.5) (layer "F.Cu") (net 29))
 (segment (start 122.25 91.75) (end 122.25 92.75) (width 0.5) (layer "F.Cu") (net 29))
 (segment (start 122.5 92) (end 126.75 92) (width 0.5) (layer "F.Cu") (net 29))
 (segment (start 141.64 92.61) (end 127.36 92.61) (width 0.5) (layer "B.Cu") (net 29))
 (segment (start 147.415 88.78) (end 145.47 88.78) (width 0.5) (layer "B.Cu") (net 29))
 (segment (start 145.47 88.78) (end 141.64 92.61) (width 0.5) (layer "B.Cu") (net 29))
 (segment (start 127.36 92.61) (end 126.75 92) (width 0.5) (layer "B.Cu") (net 29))
 (segment (start 126 81) (end 128.25 78.75) (width 0.5) (layer "F.Cu") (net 32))
 (segment (start 128.25 78.75) (end 145.005 78.75) (width 0.5) (layer "F.Cu") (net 32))
 (segment (start 145.005 78.75) (end 147.415 81.16) (width 0.5) (layer "F.Cu") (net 32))
 (segment (start 124.75 99.25) (end 124.75 101.0875) (width 0.25) (layer "F.Cu") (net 4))
 (segment (start 128.2875 113.75) (end 128.5375 113.5) (width 0.25) (layer "F.Cu") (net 15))
 (segment (start 128.2875 115.5875) (end 128.2875 113.75) (width 0.25) (layer "F.Cu") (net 15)))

